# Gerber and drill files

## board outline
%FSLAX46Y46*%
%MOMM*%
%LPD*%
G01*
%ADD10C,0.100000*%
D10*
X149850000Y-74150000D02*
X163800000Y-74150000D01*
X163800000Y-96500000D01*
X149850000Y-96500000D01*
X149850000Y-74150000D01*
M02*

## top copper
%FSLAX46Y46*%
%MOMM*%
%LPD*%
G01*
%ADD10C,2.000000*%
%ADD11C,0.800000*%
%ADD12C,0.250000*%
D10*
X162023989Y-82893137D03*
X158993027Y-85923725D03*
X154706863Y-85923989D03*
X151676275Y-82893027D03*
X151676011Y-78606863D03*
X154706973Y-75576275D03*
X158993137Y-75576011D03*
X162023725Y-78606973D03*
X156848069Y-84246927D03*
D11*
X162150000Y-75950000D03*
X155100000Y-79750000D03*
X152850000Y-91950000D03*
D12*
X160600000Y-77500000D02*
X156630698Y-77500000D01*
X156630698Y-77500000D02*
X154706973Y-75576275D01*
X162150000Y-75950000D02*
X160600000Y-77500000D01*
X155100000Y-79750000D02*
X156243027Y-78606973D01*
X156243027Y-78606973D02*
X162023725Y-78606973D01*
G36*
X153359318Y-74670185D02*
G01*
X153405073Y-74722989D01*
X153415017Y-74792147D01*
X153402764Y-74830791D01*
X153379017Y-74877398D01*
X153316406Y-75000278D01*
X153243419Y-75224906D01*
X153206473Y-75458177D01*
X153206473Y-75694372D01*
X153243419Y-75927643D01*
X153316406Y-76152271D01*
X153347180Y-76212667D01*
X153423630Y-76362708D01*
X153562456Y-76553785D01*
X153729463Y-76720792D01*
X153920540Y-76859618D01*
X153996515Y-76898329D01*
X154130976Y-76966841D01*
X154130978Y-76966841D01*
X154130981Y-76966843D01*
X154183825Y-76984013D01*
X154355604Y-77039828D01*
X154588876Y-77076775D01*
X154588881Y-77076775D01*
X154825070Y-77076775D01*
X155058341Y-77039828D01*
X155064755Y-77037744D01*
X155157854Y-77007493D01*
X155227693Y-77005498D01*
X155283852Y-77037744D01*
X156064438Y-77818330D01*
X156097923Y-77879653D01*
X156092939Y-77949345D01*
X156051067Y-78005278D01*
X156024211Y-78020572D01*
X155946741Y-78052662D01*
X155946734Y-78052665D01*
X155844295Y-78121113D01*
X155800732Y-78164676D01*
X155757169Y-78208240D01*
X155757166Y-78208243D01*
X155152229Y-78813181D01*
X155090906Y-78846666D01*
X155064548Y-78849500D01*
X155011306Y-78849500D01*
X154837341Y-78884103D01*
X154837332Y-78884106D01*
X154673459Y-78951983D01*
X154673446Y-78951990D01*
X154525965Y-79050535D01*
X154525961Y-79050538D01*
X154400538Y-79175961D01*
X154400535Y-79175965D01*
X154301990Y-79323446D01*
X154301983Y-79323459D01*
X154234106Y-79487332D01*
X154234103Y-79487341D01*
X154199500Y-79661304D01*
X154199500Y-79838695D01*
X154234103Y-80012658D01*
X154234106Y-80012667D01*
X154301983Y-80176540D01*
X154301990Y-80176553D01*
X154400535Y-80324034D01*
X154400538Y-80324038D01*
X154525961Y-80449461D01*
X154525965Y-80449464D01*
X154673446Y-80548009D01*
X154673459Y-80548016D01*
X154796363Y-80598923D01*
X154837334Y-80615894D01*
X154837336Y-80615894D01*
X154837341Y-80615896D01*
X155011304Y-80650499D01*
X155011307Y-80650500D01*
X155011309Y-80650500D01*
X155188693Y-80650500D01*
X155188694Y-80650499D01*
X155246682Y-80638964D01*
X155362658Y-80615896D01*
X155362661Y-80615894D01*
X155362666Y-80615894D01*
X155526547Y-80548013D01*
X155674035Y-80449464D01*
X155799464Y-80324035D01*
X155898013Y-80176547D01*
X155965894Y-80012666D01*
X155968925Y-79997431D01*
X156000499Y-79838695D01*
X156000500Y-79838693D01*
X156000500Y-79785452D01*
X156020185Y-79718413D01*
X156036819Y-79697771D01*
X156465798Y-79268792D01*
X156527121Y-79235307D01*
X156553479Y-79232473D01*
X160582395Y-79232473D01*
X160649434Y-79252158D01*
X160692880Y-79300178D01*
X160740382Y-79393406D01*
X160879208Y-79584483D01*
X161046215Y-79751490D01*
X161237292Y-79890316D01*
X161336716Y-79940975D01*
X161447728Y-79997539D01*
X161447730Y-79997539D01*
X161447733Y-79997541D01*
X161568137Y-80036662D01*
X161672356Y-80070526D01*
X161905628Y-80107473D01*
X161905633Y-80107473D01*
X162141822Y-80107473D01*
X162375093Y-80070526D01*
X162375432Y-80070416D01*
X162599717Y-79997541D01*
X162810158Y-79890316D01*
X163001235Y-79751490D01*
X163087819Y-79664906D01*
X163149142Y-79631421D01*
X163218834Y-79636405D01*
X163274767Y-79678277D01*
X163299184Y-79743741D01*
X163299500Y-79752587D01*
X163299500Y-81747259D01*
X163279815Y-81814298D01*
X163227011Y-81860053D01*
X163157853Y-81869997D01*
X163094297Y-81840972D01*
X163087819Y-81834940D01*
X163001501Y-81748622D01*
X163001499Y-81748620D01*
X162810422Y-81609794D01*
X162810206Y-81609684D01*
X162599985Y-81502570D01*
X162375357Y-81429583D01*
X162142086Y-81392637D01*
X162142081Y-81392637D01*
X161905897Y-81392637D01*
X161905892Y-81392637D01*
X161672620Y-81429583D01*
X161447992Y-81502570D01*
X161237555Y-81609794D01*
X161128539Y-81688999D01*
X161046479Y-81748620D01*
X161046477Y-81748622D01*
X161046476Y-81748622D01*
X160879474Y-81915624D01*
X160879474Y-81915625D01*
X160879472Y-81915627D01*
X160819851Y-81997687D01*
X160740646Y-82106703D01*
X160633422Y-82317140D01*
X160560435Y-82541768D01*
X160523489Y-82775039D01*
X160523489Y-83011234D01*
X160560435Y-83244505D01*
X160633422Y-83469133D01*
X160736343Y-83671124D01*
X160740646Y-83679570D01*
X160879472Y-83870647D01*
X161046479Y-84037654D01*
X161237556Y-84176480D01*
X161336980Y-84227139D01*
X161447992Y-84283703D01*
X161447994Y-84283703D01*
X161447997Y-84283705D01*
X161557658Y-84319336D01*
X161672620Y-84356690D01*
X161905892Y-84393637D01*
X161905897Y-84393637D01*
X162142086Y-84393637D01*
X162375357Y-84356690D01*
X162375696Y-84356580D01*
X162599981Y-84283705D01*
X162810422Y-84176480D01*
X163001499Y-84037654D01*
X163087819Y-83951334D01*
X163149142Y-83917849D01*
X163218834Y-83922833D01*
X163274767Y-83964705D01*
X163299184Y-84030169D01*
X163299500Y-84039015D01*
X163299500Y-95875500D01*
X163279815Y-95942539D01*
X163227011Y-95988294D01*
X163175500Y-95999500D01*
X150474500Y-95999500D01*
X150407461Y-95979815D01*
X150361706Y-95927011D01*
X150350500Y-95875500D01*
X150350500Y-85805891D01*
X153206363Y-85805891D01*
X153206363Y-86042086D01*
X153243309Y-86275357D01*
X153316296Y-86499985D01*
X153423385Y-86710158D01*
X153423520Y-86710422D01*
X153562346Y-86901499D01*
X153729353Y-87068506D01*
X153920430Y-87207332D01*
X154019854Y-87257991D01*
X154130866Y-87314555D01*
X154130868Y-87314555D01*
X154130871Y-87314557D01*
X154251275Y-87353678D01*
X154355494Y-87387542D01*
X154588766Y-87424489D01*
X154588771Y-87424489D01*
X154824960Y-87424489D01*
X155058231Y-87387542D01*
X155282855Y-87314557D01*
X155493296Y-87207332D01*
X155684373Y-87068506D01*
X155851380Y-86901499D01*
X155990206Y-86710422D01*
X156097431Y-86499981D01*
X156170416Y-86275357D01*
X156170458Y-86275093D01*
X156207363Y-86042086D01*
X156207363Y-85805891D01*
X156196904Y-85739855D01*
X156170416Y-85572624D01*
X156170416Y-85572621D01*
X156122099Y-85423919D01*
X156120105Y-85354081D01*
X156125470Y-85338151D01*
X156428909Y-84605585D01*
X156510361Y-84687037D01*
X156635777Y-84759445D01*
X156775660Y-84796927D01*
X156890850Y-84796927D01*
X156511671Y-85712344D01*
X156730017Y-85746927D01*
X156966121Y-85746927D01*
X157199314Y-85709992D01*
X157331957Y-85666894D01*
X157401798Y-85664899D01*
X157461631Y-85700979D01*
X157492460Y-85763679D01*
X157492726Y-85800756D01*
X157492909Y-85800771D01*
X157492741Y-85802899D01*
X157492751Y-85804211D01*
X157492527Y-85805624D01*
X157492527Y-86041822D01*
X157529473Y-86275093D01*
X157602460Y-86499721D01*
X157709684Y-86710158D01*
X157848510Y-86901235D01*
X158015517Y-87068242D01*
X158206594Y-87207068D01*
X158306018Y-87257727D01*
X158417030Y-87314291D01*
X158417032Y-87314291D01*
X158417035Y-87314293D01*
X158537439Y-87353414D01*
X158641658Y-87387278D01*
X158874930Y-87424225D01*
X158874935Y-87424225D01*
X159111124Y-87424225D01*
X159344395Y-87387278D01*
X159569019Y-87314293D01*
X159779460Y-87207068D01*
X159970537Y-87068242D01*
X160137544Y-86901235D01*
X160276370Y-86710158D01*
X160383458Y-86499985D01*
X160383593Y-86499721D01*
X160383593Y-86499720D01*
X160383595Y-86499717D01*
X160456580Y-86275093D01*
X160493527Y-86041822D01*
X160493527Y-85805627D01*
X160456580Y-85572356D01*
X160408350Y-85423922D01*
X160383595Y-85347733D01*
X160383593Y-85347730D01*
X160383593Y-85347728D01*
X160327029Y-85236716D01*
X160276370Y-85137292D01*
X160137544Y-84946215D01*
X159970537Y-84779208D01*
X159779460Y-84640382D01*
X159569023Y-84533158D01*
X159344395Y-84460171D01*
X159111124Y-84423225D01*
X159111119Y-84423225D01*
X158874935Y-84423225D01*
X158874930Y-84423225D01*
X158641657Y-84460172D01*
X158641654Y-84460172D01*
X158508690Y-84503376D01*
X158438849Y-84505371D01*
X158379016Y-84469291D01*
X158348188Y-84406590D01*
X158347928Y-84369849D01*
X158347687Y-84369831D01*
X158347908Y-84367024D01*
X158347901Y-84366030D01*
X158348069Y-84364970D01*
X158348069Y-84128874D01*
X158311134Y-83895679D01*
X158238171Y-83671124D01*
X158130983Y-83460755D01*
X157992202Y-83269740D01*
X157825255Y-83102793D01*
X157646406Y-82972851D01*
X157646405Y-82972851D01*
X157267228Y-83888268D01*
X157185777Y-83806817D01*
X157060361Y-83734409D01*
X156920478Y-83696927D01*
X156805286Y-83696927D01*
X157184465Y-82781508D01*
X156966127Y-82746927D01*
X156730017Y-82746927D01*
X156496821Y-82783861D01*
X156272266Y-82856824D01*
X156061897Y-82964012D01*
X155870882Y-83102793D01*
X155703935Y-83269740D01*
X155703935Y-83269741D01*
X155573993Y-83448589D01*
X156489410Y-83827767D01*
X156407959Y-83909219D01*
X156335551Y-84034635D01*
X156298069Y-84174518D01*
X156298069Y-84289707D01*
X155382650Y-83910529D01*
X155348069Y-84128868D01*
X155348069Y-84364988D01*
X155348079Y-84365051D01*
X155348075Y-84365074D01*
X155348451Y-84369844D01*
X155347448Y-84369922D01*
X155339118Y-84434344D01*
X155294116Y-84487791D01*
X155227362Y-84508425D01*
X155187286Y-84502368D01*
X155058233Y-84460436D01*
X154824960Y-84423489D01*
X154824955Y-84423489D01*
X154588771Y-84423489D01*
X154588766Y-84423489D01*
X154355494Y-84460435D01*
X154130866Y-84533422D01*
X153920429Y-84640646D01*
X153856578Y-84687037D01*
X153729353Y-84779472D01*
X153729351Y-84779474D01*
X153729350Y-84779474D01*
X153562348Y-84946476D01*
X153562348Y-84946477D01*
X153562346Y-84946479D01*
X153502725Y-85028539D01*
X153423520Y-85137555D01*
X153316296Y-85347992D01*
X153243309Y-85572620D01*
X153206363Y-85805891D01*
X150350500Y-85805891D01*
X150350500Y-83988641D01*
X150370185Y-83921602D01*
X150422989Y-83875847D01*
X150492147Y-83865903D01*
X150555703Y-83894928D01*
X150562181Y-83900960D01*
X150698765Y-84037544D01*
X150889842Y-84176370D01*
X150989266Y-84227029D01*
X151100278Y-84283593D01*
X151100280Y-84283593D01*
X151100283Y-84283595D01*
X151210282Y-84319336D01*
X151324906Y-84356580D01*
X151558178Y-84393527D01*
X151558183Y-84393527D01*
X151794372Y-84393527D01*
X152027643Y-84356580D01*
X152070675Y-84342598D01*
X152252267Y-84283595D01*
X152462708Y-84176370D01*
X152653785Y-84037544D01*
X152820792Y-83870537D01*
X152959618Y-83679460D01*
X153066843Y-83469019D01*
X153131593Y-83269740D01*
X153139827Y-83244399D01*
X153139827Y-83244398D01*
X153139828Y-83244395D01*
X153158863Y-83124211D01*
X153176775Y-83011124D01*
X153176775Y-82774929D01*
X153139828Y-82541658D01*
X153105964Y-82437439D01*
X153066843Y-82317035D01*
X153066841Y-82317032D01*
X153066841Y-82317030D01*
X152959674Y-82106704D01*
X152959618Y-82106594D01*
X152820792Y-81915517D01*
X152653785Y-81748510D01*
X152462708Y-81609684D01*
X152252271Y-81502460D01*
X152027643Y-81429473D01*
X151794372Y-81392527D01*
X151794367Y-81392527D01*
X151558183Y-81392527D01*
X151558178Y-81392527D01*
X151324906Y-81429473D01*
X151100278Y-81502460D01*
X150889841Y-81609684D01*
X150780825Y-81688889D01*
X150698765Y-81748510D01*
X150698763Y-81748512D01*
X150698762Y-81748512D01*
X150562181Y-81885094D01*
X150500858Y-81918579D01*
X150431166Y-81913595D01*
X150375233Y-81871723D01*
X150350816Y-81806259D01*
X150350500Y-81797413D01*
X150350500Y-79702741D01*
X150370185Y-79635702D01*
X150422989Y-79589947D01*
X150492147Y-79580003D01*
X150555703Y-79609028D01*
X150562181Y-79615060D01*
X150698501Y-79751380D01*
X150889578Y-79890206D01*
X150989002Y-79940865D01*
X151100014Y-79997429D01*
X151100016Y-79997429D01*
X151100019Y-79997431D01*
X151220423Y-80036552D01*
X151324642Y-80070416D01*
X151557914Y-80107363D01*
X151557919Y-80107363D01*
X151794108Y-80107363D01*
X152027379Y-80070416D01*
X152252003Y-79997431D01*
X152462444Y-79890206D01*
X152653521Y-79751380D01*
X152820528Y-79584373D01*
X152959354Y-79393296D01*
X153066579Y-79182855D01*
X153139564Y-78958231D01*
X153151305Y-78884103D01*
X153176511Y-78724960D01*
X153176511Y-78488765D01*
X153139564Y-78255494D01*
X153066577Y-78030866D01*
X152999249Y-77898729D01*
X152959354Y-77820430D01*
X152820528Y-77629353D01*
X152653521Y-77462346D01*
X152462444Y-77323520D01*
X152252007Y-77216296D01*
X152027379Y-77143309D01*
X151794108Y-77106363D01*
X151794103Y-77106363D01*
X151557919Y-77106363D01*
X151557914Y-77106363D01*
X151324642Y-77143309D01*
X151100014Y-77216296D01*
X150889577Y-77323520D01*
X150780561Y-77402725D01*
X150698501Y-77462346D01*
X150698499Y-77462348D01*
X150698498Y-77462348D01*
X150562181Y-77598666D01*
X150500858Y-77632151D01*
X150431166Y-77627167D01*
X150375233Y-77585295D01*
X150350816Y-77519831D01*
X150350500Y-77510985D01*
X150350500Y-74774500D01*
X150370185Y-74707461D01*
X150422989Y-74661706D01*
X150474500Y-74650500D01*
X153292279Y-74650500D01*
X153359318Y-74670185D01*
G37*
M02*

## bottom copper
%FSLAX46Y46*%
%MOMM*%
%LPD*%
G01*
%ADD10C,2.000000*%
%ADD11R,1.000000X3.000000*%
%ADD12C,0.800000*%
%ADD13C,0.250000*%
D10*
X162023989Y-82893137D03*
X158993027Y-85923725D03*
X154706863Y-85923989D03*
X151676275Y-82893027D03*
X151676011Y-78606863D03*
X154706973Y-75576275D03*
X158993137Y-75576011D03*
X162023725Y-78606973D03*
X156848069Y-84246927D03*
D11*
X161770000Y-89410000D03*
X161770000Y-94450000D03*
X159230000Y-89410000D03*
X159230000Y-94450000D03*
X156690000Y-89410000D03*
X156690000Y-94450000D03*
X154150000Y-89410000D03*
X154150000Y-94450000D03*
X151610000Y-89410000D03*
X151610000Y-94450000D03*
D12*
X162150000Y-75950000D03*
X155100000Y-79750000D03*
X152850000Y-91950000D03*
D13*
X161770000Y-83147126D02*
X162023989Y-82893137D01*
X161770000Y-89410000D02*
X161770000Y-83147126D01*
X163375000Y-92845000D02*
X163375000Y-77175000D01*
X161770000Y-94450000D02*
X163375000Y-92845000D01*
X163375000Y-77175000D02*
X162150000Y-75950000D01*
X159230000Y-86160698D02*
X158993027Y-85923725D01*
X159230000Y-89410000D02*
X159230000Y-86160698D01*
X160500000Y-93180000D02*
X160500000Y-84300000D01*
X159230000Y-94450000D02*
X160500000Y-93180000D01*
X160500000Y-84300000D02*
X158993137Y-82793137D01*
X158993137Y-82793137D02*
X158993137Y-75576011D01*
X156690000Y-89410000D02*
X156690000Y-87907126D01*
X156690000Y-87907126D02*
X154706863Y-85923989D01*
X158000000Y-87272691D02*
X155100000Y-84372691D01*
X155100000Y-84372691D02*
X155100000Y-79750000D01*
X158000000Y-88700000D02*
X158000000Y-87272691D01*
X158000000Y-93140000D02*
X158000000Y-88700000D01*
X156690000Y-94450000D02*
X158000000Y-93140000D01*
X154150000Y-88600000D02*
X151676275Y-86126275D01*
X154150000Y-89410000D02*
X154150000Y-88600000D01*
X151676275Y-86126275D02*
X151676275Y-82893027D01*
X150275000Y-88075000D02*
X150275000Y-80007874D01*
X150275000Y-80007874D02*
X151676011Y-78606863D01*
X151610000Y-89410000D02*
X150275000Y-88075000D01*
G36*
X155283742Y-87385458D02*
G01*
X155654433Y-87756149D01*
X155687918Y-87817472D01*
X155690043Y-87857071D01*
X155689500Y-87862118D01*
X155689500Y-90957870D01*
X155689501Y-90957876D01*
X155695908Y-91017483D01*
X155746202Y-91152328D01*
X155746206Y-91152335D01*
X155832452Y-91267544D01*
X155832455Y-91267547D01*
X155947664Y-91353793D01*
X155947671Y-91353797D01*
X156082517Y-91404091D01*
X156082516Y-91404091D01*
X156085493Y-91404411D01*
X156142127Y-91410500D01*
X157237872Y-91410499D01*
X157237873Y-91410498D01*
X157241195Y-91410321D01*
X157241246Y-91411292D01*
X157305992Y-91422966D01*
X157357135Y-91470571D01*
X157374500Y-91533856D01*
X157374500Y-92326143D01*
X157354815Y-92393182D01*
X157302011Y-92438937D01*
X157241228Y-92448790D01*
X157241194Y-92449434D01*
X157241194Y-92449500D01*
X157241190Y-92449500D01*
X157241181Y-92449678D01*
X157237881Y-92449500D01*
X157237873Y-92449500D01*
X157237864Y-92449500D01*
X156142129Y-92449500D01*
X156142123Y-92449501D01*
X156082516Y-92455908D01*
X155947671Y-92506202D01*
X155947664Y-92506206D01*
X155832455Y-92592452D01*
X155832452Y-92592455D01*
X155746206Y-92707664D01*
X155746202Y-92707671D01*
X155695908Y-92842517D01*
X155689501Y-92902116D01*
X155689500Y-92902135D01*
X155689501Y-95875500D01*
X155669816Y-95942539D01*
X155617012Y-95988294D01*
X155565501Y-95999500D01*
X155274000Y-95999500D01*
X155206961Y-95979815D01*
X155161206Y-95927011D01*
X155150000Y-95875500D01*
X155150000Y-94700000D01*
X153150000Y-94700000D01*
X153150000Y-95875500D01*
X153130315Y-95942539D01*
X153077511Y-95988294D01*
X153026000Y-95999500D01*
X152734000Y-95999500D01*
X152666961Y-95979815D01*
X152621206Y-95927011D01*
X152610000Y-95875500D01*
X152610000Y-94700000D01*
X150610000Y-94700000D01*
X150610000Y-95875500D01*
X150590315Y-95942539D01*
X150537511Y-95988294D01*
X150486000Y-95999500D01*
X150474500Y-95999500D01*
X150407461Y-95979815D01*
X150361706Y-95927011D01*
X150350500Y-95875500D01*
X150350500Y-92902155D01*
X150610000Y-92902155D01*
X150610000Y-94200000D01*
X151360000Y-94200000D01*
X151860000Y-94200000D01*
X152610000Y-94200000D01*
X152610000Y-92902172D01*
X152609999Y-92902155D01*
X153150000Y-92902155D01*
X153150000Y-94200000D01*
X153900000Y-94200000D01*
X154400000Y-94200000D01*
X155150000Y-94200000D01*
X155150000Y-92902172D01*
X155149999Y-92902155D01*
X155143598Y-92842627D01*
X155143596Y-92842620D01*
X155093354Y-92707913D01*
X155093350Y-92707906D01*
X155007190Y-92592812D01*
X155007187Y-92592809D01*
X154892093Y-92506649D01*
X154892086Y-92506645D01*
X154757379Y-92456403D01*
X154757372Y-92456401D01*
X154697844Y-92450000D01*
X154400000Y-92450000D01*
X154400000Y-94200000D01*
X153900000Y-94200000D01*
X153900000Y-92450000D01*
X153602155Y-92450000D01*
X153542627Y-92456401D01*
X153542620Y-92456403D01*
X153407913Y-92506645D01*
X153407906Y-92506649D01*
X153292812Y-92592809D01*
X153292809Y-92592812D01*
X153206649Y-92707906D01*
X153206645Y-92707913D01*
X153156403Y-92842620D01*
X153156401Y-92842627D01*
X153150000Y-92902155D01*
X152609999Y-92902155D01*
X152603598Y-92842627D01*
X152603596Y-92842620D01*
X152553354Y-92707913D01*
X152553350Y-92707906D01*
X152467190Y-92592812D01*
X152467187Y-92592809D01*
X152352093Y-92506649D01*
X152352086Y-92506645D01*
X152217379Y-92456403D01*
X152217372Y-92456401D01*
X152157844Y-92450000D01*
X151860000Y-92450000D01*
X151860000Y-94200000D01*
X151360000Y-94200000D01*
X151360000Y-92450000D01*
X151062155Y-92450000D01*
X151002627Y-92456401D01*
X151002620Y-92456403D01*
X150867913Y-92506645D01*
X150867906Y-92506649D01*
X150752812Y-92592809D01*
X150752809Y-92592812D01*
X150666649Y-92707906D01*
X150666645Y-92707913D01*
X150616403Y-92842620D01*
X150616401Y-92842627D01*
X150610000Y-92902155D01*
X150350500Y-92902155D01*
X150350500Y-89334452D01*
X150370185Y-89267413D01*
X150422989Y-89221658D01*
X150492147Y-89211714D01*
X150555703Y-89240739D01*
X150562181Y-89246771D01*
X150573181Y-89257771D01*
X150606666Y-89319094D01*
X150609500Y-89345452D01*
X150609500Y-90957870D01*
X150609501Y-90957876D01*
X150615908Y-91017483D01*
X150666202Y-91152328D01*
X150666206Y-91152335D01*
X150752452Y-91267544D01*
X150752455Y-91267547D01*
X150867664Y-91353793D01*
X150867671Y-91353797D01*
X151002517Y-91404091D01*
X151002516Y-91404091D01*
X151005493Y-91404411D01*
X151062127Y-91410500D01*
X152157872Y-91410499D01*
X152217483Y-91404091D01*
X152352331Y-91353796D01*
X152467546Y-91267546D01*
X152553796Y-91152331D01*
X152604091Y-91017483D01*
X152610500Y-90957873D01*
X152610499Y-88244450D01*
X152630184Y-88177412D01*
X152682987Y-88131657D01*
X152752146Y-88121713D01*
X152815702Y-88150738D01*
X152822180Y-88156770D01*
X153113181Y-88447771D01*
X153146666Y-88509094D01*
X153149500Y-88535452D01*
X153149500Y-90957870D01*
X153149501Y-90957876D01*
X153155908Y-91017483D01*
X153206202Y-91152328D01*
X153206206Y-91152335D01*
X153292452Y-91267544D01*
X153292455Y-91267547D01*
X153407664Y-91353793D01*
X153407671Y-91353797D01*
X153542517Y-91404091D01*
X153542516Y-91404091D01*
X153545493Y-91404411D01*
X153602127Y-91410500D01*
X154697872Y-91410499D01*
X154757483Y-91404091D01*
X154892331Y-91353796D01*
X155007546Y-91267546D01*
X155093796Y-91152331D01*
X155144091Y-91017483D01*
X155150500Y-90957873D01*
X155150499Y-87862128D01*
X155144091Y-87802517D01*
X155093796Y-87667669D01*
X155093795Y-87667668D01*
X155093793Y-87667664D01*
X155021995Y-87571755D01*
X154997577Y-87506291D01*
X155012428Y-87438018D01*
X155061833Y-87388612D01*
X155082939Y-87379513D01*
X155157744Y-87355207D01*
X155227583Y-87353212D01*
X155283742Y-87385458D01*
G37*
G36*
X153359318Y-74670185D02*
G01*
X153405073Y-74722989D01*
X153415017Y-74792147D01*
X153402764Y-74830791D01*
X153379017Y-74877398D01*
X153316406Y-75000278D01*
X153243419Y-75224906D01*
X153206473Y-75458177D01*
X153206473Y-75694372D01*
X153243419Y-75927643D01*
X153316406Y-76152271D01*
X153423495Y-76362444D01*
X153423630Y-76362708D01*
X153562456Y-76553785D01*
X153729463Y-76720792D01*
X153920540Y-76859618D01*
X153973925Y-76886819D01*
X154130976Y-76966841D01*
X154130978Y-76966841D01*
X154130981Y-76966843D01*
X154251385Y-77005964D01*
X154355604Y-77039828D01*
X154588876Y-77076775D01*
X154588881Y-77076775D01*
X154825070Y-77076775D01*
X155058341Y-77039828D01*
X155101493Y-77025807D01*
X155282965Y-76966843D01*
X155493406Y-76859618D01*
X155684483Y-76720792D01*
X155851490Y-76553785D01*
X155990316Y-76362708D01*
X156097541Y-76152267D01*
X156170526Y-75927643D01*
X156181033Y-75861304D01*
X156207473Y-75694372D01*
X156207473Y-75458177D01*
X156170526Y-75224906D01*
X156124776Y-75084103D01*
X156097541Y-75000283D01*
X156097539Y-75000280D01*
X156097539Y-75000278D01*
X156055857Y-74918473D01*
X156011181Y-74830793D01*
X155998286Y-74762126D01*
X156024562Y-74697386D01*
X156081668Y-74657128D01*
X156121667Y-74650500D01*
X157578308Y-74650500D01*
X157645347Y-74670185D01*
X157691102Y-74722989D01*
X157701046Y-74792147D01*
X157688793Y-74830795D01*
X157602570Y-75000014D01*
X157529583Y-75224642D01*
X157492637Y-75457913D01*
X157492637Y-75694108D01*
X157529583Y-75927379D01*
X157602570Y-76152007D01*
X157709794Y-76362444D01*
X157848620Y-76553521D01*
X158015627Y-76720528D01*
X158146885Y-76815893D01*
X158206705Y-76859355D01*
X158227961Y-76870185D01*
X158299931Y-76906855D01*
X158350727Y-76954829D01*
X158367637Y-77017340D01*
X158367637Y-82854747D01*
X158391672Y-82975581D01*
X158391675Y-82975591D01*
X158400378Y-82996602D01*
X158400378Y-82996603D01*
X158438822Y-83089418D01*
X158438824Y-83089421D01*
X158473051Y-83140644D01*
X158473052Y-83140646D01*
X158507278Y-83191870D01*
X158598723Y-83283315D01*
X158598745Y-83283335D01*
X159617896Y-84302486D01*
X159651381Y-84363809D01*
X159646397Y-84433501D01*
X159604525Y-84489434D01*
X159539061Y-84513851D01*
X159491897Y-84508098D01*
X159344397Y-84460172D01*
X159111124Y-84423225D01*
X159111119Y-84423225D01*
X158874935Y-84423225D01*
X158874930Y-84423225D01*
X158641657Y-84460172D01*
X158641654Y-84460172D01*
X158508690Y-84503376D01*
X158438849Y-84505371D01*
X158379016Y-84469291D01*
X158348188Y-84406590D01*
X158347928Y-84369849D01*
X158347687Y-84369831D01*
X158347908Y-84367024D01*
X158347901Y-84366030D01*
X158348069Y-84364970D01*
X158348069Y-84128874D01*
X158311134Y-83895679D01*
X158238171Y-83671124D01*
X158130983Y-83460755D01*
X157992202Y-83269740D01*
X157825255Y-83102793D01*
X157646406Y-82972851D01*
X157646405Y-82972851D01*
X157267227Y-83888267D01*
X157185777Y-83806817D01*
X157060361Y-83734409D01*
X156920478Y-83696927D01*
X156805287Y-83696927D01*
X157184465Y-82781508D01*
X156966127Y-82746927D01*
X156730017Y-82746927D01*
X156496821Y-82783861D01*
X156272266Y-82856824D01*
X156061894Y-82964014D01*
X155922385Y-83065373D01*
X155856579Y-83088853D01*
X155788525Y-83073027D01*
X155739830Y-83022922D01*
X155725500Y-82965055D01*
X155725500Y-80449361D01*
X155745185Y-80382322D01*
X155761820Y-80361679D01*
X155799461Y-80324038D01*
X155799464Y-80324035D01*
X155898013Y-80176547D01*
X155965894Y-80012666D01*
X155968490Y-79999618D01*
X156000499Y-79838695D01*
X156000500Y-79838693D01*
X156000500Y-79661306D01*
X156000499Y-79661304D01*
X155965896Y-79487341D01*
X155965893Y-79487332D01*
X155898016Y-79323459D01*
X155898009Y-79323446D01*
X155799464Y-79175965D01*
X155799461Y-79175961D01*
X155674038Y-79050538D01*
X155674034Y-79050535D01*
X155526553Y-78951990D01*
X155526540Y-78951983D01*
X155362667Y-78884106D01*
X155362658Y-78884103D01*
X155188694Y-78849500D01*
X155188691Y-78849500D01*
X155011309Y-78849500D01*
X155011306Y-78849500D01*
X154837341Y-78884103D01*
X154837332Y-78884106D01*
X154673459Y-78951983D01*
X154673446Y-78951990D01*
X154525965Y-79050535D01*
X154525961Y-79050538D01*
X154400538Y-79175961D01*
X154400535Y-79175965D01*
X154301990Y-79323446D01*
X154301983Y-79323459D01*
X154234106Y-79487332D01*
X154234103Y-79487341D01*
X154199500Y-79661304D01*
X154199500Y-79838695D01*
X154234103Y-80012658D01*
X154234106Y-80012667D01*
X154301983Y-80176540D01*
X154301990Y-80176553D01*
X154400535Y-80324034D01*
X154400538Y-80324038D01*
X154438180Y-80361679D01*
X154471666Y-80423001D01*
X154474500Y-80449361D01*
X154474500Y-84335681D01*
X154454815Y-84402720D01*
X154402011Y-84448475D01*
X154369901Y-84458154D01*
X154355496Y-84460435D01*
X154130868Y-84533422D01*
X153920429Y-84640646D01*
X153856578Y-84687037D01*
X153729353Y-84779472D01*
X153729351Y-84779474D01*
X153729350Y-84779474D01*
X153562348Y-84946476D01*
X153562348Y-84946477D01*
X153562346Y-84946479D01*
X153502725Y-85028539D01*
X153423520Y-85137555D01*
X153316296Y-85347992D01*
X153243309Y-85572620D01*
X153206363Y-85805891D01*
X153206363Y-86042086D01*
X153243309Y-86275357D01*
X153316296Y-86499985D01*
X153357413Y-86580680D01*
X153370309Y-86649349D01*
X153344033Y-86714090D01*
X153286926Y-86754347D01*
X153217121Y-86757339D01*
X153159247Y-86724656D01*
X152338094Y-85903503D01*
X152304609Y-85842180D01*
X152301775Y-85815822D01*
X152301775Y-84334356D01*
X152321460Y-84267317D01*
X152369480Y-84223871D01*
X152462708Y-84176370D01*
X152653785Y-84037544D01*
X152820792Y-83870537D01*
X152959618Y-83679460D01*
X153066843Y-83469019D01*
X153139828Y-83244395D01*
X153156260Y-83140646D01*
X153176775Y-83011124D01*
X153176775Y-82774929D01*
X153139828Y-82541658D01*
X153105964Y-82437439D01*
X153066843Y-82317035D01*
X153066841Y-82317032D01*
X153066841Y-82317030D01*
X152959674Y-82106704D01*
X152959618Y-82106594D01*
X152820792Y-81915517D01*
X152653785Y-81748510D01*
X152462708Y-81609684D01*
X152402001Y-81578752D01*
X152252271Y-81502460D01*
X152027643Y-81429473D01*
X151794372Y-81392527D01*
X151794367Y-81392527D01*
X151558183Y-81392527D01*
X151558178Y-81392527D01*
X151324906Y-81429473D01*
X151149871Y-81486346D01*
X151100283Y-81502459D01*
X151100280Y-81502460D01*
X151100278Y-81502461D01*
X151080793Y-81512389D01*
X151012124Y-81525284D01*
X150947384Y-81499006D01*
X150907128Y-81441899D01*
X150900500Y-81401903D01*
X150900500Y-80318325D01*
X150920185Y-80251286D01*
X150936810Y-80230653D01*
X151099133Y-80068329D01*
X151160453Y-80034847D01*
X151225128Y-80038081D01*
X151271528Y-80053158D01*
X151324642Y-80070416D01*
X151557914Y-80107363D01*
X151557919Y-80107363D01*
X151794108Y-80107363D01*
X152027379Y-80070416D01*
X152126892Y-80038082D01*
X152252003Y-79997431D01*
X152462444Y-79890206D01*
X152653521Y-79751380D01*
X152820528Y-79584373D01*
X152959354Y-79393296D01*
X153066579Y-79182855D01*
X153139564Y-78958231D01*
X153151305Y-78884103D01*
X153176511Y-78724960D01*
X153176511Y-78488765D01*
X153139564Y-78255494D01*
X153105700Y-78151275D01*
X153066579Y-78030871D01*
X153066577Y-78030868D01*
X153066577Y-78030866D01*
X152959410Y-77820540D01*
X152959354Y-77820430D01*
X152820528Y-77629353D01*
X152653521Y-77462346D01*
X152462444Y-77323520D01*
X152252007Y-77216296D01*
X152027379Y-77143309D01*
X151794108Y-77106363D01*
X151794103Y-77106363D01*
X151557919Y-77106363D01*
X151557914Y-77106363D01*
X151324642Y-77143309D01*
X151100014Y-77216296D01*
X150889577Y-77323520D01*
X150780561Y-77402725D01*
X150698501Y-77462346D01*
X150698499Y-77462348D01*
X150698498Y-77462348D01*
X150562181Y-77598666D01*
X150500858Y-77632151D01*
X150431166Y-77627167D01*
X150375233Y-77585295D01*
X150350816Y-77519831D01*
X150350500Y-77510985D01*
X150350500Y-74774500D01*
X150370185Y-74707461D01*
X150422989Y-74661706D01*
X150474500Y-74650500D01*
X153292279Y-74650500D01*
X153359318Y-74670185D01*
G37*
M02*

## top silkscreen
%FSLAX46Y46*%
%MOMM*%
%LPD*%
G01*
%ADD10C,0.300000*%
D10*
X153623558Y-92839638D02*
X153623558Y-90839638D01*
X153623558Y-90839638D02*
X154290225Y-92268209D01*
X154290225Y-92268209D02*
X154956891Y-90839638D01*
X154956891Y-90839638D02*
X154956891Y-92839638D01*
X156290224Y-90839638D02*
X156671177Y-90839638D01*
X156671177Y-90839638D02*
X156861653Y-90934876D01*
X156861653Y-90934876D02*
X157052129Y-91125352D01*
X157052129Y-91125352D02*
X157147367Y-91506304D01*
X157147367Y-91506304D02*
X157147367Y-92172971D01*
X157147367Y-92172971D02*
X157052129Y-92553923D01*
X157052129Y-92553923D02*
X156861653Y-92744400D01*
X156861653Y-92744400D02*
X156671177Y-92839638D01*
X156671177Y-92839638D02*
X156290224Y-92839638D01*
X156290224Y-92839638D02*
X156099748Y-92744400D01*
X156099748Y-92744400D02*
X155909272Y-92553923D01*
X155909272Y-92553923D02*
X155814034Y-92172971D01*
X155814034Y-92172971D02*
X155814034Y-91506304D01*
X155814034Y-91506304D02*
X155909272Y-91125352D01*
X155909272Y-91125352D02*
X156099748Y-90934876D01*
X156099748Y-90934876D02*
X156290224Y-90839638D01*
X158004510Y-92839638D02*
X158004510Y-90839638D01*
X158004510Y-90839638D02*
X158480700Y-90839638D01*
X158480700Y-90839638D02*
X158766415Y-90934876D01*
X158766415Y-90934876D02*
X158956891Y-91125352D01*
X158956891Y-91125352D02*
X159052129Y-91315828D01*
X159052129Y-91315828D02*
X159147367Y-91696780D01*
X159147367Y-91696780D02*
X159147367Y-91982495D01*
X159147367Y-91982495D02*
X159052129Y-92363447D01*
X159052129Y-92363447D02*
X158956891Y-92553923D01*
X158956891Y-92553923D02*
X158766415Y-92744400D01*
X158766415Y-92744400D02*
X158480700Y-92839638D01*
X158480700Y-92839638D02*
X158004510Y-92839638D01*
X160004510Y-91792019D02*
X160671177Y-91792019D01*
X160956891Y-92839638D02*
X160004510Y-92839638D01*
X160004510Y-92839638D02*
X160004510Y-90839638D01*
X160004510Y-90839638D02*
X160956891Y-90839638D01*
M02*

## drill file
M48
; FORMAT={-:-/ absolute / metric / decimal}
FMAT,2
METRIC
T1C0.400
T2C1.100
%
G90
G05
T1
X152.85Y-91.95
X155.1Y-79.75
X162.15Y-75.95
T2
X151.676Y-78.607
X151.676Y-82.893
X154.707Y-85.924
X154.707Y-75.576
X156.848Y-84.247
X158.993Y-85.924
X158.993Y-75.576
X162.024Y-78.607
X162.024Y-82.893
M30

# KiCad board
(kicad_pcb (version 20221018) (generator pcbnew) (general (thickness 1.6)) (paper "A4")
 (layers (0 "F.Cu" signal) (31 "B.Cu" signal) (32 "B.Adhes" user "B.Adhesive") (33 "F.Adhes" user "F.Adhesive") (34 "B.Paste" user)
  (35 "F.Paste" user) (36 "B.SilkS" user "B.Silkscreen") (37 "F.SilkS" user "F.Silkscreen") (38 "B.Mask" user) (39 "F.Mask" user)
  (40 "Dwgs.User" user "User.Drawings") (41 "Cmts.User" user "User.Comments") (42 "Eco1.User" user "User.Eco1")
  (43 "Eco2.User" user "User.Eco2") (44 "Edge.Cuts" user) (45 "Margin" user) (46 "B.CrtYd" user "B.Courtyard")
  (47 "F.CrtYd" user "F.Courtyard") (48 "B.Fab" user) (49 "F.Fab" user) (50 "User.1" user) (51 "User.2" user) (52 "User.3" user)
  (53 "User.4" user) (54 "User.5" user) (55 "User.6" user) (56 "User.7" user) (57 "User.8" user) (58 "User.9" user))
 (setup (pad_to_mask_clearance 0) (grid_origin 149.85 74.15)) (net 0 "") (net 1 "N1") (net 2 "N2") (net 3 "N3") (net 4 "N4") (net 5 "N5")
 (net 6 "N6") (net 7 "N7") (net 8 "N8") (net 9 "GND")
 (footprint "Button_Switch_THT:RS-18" (layer "F.Cu") (at 156.85 80.75 112.5)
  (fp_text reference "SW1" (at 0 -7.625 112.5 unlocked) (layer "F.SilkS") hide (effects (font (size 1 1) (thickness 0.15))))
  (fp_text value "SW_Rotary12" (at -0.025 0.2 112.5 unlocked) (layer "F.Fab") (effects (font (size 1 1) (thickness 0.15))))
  (pad "1" thru_hole circle (at -3.96 3.96 112.5) (size 2 2) (drill 1.1) (layers "*.Cu" "*.Mask") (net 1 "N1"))
  (pad "2" thru_hole circle (at -5.6 0 112.5) (size 2 2) (drill 1.1) (layers "*.Cu" "*.Mask") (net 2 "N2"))
  (pad "3" thru_hole circle (at -3.96 -3.96 112.5) (size 2 2) (drill 1.1) (layers "*.Cu" "*.Mask") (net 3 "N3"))
  (pad "4" thru_hole circle (at 0 -5.6 112.5) (size 2 2) (drill 1.1) (layers "*.Cu" "*.Mask") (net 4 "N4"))
  (pad "5" thru_hole circle (at 3.96 -3.96 112.5) (size 2 2) (drill 1.1) (layers "*.Cu" "*.Mask") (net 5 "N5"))
  (pad "6" thru_hole circle (at 5.6 0 112.5) (size 2 2) (drill 1.1) (layers "*.Cu" "*.Mask") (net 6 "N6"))
  (pad "7" thru_hole circle (at 3.96 3.96 112.5) (size 2 2) (drill 1.1) (layers "*.Cu" "*.Mask") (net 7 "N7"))
  (pad "8" thru_hole circle (at 0 5.6 112.5) (size 2 2) (drill 1.1) (layers "*.Cu" "*.Mask") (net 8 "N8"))
  (pad "C" thru_hole circle (at -3.23 -1.34 112.5) (size 2 2) (drill 1.1) (layers "*.Cu" "*.Mask") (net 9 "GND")))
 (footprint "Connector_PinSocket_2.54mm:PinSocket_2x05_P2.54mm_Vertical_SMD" (layer "B.Cu") (at 156.69 91.93 90)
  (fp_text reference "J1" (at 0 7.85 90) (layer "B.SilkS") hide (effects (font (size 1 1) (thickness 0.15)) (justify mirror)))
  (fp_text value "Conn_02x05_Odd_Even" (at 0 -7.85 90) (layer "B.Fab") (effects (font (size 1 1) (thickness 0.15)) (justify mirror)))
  (pad "1" smd rect (at 2.52 5.08 90) (size 3 1) (layers "B.Cu" "B.Paste" "B.Mask") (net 1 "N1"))
  (pad "2" smd rect (at -2.52 5.08 90) (size 3 1) (layers "B.Cu" "B.Paste" "B.Mask") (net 6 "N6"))
  (pad "3" smd rect (at 2.52 2.54 90) (size 3 1) (layers "B.Cu" "B.Paste" "B.Mask") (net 2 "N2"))
  (pad "4" smd rect (at -2.52 2.54 90) (size 3 1) (layers "B.Cu" "B.Paste" "B.Mask") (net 7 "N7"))
  (pad "5" smd rect (at 2.52 0 90) (size 3 1) (layers "B.Cu" "B.Paste" "B.Mask") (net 3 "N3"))
  (pad "6" smd rect (at -2.52 0 90) (size 3 1) (layers "B.Cu" "B.Paste" "B.Mask") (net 8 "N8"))
  (pad "7" smd rect (at 2.52 -2.54 90) (size 3 1) (layers "B.Cu" "B.Paste" "B.Mask") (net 4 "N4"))
  (pad "8" smd rect (at -2.52 -2.54 90) (size 3 1) (layers "B.Cu" "B.Paste" "B.Mask") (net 9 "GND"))
  (pad "9" smd rect (at 2.52 -5.08 90) (size 3 1) (layers "B.Cu" "B.Paste" "B.Mask") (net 5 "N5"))
  (pad "10" smd rect (at -2.52 -5.08 90) (size 3 1) (layers "B.Cu" "B.Paste" "B.Mask") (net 9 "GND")))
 (gr_rect (start 149.85 74.15) (end 163.8 96.5) (stroke (width 0.1) (type default)) (fill none) (layer "Edge.Cuts"))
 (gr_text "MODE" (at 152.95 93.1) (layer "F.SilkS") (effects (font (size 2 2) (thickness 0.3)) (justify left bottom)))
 (segment (start 161.77 83.147126) (end 162.023989 82.893137) (width 0.25) (layer "B.Cu") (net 1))
 (segment (start 161.77 89.41) (end 161.77 83.147126) (width 0.25) (layer "B.Cu") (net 1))
 (segment (start 160.6 77.5) (end 156.630698 77.5) (width 0.25) (layer "F.Cu") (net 6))
 (segment (start 156.630698 77.5) (end 154.706973 75.576275) (width 0.25) (layer "F.Cu") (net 6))
 (segment (start 162.15 75.95) (end 160.6 77.5) (width 0.25) (layer "F.Cu") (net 6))
 (via (at 162.15 75.95) (size 0.8) (drill 0.4) (layers "F.Cu" "B.Cu") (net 6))
 (segment (start 163.375 92.845) (end 163.375 77.175) (width 0.25) (layer "B.Cu") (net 6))
 (segment (start 161.77 94.45) (end 163.375 92.845) (width 0.25) (layer "B.Cu") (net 6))
 (segment (start 163.375 77.175) (end 162.15 75.95) (width 0.25) (layer "B.Cu") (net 6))
 (segment (start 159.23 86.160698) (end 158.993027 85.923725) (width 0.25) (layer "B.Cu") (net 2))
 (segment (start 159.23 89.41) (end 159.23 86.160698) (width 0.25) (layer "B.Cu") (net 2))
 (segment (start 160.5 93.18) (end 160.5 84.3) (width 0.25) (layer "B.Cu") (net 7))
 (segment (start 159.23 94.45) (end 160.5 93.18) (width 0.25) (layer "B.Cu") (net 7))
 (segment (start 160.5 84.3) (end 158.993137 82.793137) (width 0.25) (layer "B.Cu") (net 7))
 (segment (start 158.993137 82.793137) (end 158.993137 75.576011) (width 0.25) (layer "B.Cu") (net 7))
 (segment (start 156.69 89.41) (end 156.69 87.907126) (width 0.25) (layer "B.Cu") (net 3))
 (segment (start 156.69 87.907126) (end 154.706863 85.923989) (width 0.25) (layer "B.Cu") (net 3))
 (segment (start 155.1 79.75) (end 156.243027 78.606973) (width 0.25) (layer "F.Cu") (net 8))
 (segment (start 156.243027 78.606973) (end 162.023725 78.606973) (width 0.25) (layer "F.Cu") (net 8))
 (via (at 155.1 79.75) (size 0.8) (drill 0.4) (layers "F.Cu" "B.Cu") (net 8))
 (segment (start 158 87.272691) (end 155.1 84.372691) (width 0.25) (layer "B.Cu") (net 8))
 (segment (start 155.1 84.372691) (end 155.1 79.75) (width 0.25) (layer "B.Cu") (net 8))
 (segment (start 158 88.7) (end 158 87.272691) (width 0.25) (layer "B.Cu") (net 8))
 (segment (start 158 93.14) (end 158 88.7) (width 0.25) (layer "B.Cu") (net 8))
 (segment (start 156.69 94.45) (end 158 93.14) (width 0.25) (layer "B.Cu") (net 8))
 (segment (start 154.15 88.6) (end 151.676275 86.126275) (width 0.25) (layer "B.Cu") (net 4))
 (segment (start 154.15 89.41) (end 154.15 88.6) (width 0.25) (layer "B.Cu") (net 4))
 (segment (start 151.676275 86.126275) (end 151.676275 82.893027) (width 0.25) (layer "B.Cu") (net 4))
 (via (at 152.85 91.95) (size 0.8) (drill 0.4) (layers "F.Cu" "B.Cu") (free) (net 9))
 (segment (start 150.275 88.075) (end 150.275 80.007874) (width 0.25) (layer "B.Cu") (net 5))
 (segment (start 150.275 80.007874) (end 151.676011 78.606863) (width 0.25) (layer "B.Cu") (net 5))
 (segment (start 151.61 89.41) (end 150.275 88.075) (width 0.25) (layer "B.Cu") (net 5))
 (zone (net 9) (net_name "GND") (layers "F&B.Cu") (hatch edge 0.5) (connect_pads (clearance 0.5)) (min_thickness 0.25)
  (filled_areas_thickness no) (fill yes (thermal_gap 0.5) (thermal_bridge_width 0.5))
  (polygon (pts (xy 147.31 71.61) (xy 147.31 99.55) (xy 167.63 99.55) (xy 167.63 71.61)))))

